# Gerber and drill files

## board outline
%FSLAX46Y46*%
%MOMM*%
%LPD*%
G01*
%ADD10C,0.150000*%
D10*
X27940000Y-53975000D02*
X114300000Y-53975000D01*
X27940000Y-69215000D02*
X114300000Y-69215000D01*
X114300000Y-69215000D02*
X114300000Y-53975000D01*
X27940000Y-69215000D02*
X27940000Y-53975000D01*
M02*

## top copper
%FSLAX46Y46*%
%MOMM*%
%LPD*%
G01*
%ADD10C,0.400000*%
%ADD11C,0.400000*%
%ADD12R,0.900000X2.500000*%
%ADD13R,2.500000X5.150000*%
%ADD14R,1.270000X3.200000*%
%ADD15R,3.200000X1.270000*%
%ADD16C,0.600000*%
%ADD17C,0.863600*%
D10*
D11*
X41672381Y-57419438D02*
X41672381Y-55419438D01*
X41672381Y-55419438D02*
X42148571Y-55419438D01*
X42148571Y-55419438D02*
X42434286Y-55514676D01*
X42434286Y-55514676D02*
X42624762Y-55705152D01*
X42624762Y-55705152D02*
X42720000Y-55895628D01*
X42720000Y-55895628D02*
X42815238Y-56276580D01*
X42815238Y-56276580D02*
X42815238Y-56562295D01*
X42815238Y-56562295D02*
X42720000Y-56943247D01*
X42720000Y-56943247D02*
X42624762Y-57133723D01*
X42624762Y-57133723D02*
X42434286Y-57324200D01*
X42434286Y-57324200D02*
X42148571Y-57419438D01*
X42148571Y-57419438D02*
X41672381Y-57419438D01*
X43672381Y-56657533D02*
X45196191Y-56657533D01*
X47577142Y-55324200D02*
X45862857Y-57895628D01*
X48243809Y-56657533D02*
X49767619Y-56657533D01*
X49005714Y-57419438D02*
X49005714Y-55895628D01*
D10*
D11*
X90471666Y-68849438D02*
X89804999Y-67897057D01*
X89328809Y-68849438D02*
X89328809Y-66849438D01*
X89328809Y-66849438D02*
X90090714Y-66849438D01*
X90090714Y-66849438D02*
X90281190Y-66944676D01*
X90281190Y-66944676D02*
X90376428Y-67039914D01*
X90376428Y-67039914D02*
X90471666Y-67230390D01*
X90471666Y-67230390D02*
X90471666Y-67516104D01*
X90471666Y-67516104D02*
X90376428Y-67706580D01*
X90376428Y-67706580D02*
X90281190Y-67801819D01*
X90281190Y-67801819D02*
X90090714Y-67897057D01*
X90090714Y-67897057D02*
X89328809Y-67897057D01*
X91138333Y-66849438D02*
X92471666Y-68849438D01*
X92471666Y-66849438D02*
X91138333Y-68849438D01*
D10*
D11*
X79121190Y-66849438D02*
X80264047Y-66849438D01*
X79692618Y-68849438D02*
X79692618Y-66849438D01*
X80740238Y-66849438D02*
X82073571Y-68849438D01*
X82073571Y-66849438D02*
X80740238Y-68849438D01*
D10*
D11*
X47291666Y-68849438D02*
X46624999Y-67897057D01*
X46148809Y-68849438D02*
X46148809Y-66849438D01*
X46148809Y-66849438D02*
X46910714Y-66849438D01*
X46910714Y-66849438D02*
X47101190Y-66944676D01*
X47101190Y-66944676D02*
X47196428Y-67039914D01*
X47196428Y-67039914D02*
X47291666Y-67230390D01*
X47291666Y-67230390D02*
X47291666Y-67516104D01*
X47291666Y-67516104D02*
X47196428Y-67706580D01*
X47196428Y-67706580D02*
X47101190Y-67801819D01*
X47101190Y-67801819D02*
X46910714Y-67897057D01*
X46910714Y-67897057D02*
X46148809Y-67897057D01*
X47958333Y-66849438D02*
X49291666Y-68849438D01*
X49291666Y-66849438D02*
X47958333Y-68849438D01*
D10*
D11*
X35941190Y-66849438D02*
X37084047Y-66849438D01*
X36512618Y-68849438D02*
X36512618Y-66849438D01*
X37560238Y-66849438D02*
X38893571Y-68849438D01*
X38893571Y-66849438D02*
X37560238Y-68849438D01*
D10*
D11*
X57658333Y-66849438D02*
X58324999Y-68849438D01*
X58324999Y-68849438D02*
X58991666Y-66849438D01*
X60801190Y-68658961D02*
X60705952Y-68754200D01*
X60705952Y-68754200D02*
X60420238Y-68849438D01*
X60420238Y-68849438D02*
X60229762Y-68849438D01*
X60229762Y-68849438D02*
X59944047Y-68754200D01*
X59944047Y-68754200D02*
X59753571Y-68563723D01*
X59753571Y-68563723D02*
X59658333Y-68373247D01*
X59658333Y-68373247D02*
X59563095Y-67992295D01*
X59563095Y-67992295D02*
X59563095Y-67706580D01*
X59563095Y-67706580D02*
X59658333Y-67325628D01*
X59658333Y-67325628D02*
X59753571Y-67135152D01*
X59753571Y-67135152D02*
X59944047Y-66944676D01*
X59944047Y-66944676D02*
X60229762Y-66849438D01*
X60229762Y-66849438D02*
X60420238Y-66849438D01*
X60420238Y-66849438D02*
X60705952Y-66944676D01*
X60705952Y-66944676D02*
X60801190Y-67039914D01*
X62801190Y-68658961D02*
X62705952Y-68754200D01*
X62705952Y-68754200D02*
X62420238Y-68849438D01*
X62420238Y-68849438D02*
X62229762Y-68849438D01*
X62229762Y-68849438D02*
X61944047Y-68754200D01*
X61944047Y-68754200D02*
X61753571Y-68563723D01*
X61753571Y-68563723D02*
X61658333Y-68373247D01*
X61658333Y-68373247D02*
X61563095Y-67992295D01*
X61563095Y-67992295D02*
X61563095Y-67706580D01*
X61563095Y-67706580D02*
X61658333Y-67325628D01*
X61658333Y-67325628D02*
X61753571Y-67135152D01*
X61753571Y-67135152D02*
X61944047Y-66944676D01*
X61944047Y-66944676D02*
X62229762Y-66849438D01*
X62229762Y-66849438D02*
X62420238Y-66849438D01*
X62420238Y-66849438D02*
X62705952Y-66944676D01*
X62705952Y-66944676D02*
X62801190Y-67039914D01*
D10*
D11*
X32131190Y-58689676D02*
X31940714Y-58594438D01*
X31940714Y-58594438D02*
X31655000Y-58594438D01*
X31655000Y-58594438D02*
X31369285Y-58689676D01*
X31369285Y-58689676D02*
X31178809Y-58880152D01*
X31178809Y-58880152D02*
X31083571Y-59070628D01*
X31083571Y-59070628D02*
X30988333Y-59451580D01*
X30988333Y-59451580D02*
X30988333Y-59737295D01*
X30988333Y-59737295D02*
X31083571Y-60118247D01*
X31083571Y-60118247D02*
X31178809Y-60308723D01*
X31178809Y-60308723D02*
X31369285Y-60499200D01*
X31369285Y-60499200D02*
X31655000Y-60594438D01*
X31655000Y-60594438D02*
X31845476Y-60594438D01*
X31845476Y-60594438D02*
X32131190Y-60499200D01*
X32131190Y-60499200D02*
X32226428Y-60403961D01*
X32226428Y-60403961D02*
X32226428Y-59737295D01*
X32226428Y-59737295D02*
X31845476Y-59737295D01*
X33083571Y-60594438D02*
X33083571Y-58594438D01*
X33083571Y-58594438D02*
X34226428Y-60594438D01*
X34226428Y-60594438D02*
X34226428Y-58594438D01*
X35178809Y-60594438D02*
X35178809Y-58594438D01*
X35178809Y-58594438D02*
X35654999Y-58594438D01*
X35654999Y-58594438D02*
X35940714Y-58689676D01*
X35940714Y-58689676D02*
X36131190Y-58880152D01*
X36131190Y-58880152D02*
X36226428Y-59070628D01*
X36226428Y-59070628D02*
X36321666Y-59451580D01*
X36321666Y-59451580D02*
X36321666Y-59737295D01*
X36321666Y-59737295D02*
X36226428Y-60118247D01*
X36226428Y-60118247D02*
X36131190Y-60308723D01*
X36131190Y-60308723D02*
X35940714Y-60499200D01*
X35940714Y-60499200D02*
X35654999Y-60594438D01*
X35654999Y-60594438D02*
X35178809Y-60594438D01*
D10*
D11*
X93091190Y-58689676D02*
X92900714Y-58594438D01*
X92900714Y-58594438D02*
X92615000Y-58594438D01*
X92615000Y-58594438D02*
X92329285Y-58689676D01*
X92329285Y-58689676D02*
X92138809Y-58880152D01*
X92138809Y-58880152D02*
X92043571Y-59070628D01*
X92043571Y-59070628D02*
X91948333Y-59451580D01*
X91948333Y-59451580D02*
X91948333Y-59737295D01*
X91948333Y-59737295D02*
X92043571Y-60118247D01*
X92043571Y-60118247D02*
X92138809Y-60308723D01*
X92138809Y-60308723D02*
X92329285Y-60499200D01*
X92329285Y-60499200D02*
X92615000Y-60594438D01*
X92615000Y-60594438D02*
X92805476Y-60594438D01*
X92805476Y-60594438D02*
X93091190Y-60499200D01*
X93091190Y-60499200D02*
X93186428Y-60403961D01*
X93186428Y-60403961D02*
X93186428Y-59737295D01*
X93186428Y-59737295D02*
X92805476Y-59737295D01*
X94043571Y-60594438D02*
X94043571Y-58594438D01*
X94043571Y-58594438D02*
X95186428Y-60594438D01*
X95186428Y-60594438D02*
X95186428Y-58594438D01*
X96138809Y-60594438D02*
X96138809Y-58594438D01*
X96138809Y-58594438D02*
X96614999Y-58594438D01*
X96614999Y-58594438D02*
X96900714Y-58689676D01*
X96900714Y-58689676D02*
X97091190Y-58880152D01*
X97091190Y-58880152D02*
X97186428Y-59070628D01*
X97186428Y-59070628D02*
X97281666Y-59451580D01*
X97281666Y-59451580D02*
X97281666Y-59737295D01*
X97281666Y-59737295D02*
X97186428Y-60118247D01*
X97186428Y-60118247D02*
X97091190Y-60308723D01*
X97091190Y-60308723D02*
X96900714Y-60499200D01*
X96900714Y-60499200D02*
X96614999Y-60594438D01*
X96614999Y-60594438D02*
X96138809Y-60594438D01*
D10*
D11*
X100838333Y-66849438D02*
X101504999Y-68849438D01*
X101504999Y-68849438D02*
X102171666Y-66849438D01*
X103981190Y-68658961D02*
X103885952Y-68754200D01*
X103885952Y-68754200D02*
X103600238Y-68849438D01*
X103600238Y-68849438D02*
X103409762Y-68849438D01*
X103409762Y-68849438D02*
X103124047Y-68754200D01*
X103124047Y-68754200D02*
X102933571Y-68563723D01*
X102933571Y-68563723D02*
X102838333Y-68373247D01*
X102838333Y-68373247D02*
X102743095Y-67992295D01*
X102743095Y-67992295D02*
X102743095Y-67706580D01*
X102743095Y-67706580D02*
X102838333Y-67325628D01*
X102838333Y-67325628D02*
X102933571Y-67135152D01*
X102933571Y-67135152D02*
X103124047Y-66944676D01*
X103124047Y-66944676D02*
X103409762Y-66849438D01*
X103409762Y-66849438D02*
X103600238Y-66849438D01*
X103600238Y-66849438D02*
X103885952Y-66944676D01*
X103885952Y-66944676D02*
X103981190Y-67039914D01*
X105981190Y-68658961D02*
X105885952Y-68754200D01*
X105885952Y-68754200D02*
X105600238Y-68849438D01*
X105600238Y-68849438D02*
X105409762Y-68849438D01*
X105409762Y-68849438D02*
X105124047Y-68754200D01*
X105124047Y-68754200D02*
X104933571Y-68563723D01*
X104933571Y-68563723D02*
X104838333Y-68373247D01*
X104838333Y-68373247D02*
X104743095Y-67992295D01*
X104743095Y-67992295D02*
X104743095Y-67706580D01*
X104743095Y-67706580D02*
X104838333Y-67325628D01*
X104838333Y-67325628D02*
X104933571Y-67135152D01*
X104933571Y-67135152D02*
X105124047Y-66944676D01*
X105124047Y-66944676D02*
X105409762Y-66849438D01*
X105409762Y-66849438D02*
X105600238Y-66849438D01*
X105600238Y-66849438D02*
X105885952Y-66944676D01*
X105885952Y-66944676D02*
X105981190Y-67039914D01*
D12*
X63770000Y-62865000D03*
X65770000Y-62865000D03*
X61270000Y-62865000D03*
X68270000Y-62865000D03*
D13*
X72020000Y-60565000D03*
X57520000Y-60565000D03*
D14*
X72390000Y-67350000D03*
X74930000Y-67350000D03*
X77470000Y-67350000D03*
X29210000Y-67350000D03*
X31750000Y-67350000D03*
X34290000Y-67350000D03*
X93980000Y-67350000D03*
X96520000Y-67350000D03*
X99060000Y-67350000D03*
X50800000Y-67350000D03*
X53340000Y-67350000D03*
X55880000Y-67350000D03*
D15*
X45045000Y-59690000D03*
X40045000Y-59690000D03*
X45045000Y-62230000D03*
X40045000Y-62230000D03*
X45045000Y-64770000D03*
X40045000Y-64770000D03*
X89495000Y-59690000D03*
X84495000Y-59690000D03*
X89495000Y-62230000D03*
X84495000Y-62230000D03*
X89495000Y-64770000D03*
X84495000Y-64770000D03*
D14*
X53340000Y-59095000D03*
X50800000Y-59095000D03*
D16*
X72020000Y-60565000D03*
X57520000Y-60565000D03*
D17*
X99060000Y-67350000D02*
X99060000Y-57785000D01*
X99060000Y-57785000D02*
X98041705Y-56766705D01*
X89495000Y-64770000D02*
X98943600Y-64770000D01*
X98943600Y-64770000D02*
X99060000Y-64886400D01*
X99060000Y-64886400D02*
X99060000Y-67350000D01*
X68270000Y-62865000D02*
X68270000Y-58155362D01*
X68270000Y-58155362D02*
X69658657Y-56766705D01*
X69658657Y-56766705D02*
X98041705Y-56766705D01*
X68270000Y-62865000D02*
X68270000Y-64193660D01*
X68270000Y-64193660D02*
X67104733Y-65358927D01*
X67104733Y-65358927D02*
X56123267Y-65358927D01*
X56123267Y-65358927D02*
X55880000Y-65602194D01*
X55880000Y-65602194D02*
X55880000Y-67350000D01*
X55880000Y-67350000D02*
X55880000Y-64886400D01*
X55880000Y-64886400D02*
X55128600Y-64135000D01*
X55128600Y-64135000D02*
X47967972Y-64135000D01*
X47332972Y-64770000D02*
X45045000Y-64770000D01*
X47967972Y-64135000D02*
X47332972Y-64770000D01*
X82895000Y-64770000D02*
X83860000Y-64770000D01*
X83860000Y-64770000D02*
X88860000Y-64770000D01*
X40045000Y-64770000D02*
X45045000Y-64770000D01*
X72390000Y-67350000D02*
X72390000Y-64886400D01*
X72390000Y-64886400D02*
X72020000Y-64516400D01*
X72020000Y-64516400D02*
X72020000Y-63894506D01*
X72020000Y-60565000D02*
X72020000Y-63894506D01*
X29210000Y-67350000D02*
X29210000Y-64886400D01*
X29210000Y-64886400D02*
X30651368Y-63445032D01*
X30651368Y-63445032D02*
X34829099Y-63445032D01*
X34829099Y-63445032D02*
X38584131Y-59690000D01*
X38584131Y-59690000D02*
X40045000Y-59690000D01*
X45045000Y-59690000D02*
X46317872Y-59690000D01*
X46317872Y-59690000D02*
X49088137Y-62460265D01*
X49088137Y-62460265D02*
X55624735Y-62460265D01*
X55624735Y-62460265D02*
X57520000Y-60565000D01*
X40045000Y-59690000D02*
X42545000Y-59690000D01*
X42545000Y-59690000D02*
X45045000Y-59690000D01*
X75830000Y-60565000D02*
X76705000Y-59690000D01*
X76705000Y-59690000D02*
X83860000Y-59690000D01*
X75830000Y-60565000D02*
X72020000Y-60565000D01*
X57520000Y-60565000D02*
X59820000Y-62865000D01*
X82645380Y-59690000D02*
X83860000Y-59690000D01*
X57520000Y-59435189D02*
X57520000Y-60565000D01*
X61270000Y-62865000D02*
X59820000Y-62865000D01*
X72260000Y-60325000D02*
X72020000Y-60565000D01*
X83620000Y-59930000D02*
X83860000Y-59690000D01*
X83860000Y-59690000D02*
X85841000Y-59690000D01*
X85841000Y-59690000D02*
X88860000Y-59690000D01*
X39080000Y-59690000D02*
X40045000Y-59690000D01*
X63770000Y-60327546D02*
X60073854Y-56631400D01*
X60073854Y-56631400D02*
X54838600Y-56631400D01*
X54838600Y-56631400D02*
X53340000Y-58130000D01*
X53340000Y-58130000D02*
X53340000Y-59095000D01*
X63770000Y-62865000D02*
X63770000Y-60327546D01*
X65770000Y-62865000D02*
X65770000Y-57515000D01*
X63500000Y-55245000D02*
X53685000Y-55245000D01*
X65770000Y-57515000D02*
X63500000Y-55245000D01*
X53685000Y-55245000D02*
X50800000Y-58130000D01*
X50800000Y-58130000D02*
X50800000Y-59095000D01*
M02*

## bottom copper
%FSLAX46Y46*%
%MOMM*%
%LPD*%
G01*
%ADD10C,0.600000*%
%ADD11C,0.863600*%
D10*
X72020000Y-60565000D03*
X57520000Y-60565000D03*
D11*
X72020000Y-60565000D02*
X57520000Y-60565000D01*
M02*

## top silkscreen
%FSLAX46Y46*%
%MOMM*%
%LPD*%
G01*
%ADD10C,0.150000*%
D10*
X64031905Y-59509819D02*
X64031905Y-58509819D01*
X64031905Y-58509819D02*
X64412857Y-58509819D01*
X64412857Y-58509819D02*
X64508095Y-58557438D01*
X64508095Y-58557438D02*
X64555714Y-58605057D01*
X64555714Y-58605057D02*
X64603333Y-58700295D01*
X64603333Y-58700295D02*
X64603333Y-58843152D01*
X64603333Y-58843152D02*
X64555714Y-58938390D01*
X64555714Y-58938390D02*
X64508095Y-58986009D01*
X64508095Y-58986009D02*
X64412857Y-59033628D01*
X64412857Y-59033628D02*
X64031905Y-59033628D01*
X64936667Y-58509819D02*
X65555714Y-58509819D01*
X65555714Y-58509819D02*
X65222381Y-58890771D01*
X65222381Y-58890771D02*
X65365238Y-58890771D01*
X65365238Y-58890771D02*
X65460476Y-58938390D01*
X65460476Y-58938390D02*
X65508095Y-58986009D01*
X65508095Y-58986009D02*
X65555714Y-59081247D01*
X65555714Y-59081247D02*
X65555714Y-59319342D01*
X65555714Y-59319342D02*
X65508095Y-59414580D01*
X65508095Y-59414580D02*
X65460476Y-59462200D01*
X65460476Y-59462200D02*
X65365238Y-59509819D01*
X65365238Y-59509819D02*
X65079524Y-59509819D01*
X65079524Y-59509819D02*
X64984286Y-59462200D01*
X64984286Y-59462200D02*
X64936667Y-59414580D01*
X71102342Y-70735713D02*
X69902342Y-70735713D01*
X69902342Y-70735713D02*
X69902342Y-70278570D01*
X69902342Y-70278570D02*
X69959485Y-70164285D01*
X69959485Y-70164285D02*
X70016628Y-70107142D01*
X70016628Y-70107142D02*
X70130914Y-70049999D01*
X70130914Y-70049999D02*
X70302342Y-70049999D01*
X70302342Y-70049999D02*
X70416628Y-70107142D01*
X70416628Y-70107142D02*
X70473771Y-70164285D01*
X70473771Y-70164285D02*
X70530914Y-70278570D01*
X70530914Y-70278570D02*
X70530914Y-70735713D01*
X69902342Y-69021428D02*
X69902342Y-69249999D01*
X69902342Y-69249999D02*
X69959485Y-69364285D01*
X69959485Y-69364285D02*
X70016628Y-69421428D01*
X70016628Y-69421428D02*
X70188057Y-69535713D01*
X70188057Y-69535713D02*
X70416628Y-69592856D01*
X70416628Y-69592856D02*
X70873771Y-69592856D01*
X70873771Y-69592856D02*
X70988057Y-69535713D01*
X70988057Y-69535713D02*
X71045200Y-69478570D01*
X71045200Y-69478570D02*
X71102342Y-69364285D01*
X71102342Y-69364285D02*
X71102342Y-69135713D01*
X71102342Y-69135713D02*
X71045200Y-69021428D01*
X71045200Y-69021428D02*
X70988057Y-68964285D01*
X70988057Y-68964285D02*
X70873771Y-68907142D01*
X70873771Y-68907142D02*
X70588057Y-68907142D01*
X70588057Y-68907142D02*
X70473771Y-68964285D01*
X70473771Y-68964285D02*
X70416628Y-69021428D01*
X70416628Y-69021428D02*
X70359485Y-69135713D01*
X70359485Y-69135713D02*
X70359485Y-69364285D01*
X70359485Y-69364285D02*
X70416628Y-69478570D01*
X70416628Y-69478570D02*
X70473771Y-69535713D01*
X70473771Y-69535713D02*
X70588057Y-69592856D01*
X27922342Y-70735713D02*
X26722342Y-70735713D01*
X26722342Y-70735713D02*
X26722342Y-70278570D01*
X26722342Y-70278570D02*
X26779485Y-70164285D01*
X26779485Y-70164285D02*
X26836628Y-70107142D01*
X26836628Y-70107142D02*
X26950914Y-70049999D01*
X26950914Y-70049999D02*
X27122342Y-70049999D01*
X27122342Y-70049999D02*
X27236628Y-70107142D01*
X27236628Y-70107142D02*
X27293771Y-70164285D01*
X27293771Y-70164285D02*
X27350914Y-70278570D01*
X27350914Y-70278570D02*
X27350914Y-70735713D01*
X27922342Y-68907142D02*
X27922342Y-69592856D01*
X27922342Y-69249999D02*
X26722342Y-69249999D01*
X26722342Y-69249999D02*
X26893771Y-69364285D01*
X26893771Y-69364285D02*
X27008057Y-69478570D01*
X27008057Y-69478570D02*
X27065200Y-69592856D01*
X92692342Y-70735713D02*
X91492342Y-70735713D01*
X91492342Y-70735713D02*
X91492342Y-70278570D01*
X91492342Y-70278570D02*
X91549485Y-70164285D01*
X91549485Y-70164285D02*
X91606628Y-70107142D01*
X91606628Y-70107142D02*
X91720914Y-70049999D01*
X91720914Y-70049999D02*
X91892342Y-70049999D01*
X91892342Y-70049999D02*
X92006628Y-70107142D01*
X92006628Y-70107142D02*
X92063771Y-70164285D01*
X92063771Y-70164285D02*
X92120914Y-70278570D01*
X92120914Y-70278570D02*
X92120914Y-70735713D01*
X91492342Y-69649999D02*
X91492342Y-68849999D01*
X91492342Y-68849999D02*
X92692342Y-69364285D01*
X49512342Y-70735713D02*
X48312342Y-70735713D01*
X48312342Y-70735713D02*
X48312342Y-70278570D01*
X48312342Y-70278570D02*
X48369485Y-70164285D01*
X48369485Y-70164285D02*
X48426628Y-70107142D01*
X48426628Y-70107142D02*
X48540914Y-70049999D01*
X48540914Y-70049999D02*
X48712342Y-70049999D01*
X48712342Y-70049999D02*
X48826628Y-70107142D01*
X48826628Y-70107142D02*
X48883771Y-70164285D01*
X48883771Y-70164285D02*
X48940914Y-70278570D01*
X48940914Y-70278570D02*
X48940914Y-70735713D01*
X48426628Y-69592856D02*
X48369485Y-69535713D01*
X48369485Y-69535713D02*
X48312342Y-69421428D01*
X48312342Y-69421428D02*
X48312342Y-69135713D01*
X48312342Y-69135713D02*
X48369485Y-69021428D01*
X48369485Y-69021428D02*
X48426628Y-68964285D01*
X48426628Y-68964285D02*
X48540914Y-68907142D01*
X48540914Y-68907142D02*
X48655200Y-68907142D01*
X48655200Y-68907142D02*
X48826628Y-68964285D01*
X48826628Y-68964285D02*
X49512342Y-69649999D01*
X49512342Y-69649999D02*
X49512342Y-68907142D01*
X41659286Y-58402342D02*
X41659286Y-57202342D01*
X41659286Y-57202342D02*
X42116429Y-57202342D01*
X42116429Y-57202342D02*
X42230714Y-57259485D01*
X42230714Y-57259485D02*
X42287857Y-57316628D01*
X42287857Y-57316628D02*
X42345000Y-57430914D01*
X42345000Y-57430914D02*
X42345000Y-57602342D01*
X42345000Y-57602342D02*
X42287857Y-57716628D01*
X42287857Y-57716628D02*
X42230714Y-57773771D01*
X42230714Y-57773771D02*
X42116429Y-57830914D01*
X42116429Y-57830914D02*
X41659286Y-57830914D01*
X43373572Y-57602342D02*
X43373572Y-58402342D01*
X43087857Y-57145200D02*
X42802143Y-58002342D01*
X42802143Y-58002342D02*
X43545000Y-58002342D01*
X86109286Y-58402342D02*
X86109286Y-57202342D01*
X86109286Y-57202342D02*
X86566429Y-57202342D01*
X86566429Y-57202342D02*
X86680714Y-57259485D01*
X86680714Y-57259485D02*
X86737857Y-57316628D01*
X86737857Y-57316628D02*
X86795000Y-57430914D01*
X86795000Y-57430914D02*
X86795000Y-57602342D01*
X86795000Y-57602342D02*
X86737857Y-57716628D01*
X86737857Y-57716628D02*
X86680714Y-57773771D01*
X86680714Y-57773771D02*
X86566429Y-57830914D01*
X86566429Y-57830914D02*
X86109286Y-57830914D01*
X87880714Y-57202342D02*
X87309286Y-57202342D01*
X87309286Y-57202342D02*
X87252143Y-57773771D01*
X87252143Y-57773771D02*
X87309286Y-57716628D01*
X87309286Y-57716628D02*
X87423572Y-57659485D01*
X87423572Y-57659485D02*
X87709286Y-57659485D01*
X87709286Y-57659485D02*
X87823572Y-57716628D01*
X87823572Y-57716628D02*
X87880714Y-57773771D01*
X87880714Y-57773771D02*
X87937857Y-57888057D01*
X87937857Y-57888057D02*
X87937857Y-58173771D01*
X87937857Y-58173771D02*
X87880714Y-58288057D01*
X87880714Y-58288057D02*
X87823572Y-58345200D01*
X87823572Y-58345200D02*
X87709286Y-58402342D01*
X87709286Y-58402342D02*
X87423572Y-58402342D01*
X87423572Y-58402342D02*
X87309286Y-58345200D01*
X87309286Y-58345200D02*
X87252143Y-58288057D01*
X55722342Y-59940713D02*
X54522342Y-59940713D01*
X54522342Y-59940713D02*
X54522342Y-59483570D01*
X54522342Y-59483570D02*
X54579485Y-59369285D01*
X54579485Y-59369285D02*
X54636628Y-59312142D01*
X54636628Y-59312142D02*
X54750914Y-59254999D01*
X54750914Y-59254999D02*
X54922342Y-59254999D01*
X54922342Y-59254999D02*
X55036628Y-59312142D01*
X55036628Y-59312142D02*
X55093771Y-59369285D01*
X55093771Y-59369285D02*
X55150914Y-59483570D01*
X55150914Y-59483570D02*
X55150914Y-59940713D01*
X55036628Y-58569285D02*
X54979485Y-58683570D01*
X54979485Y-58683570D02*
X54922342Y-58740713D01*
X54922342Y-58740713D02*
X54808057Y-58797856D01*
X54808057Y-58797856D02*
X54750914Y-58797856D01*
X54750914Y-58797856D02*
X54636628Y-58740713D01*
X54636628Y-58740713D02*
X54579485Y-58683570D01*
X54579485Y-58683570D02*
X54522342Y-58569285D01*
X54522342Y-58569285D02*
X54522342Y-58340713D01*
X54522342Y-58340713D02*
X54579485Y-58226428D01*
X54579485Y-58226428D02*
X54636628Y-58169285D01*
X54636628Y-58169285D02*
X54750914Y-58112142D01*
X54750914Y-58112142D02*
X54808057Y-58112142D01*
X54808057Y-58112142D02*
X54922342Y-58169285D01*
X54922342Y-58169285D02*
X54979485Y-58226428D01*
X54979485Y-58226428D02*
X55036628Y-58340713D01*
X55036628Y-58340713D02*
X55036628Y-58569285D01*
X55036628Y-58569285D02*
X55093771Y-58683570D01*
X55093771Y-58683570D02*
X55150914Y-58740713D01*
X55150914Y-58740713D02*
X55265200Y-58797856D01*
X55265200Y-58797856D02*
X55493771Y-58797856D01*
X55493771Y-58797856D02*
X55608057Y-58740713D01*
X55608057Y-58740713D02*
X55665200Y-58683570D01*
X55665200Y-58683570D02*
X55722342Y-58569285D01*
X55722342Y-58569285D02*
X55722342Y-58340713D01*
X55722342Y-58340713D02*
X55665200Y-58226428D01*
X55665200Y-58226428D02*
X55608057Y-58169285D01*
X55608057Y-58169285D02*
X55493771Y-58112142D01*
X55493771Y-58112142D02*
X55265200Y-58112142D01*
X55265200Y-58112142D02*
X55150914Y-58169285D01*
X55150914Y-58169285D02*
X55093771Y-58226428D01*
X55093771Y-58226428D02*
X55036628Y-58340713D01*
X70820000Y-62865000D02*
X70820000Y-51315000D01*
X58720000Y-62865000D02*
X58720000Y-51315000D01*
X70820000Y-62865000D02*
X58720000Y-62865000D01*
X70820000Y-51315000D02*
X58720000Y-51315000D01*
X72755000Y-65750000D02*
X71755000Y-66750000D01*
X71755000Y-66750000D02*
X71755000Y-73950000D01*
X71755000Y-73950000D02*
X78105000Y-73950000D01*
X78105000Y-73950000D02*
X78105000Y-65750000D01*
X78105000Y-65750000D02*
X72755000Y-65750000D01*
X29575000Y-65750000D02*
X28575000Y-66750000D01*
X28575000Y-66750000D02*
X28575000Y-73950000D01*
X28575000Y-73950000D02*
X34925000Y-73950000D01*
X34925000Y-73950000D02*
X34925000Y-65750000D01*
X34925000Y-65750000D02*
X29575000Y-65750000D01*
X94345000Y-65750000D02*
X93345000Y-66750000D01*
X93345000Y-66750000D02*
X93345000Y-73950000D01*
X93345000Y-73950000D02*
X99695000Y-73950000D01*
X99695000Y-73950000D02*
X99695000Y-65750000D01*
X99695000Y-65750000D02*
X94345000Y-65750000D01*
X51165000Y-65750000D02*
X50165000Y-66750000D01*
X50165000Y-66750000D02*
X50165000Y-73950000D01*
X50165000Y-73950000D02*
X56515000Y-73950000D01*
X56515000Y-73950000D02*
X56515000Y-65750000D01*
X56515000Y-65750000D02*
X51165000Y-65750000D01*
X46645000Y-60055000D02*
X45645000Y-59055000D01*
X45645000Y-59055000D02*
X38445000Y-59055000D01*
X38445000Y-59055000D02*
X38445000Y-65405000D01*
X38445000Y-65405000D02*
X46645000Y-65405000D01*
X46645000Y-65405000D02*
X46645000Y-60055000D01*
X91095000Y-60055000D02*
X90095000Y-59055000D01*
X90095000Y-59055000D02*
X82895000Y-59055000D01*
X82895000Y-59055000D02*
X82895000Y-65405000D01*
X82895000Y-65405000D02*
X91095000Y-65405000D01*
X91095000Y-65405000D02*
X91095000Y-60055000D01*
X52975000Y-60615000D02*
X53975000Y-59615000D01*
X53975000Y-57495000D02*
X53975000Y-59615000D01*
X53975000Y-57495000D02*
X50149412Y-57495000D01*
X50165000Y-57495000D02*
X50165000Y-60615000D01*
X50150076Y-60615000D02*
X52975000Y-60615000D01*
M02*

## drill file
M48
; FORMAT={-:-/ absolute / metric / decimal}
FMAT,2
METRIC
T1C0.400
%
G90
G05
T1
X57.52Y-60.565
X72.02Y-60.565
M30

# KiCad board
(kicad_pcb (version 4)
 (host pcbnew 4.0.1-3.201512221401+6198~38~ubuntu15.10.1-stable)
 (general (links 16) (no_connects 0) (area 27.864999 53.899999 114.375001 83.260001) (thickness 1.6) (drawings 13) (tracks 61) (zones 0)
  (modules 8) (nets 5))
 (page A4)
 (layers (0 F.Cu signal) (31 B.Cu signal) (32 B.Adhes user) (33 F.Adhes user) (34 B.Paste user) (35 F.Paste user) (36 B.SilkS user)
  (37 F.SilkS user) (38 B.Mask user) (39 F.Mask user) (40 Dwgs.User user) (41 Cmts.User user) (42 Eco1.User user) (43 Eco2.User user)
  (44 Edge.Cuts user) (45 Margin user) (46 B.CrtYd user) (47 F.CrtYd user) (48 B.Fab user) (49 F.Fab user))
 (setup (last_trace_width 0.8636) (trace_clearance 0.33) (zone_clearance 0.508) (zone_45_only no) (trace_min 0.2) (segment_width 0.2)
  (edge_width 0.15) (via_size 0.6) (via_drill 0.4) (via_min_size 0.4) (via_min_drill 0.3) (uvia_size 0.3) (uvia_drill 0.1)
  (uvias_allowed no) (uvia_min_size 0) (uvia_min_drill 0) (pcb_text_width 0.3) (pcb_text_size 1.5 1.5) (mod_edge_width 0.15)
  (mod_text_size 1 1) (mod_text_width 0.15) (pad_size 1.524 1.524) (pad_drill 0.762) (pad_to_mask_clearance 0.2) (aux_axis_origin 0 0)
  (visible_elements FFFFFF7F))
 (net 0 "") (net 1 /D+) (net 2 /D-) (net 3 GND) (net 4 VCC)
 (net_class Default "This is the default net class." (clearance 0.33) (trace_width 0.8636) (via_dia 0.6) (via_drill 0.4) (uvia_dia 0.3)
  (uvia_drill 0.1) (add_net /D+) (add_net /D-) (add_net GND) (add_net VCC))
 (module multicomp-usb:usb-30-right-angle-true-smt (layer F.Cu) (at 64.77 62.865 180)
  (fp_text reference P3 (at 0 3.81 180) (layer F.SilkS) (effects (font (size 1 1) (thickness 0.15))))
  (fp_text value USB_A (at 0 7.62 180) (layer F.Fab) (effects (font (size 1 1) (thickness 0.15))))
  (fp_line (start -6.05 0) (end -6.05 11.55) (layer F.SilkS) (width 0.15))
  (fp_line (start 6.05 0) (end 6.05 11.55) (layer F.SilkS) (width 0.15))
  (fp_line (start -6.05 0) (end 6.05 0) (layer F.SilkS) (width 0.15))
  (fp_line (start -6.05 11.55) (end 6.05 11.55) (layer F.SilkS) (width 0.15))
  (pad 3 smd rect (at 1 0 180) (size 0.9 2.5) (layers F.Cu F.Paste F.Mask) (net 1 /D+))
  (pad 2 smd rect (at -1 0 180) (size 0.9 2.5) (layers F.Cu F.Paste F.Mask) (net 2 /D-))
  (pad 4 smd rect (at 3.5 0 180) (size 0.9 2.5) (layers F.Cu F.Paste F.Mask) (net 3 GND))
  (pad 1 smd rect (at -3.5 0 180) (size 0.9 2.5) (layers F.Cu F.Paste F.Mask) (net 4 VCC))
  (pad 5 smd rect (at -7.25 2.3 180) (size 2.5 5.15) (layers F.Cu F.Paste F.Mask) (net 3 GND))
  (pad 5 smd rect (at 7.25 2.3 180) (size 2.5 5.15) (layers F.Cu F.Paste F.Mask) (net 3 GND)))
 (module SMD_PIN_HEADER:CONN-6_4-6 (layer F.Cu) (at 74.93 69.85)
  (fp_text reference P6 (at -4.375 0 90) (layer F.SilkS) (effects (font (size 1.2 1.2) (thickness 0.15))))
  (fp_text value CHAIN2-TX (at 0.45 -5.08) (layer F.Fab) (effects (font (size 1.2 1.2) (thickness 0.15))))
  (fp_line (start -2.175 -4.1) (end -3.175 -3.1) (layer F.SilkS) (width 0.15))
  (fp_line (start -3.175 -3.1) (end -3.175 4.1) (layer F.SilkS) (width 0.15))
  (fp_line (start -3.175 4.1) (end 3.175 4.1) (layer F.SilkS) (width 0.15))
  (fp_line (start 3.175 4.1) (end 3.175 -4.1) (layer F.SilkS) (width 0.15))
  (fp_line (start 3.175 -4.1) (end -2.175 -4.1) (layer F.SilkS) (width 0.15))
  (pad 6 smd rect (at -2.54 -2.5) (size 1.27 3.2) (layers F.Cu F.Paste F.Mask) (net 3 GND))
  (pad 5 smd rect (at 0 -2.5) (size 1.27 3.2) (layers F.Cu F.Paste F.Mask))
  (pad 4 smd rect (at 2.54 -2.5) (size 1.27 3.2) (layers F.Cu F.Paste F.Mask)))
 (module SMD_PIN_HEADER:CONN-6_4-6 (layer F.Cu) (at 31.75 69.85)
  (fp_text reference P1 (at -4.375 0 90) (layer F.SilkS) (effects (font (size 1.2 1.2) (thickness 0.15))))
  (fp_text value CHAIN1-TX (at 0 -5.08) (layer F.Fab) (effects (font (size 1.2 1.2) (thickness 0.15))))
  (fp_line (start -2.175 -4.1) (end -3.175 -3.1) (layer F.SilkS) (width 0.15))
  (fp_line (start -3.175 -3.1) (end -3.175 4.1) (layer F.SilkS) (width 0.15))
  (fp_line (start -3.175 4.1) (end 3.175 4.1) (layer F.SilkS) (width 0.15))
  (fp_line (start 3.175 4.1) (end 3.175 -4.1) (layer F.SilkS) (width 0.15))
  (fp_line (start 3.175 -4.1) (end -2.175 -4.1) (layer F.SilkS) (width 0.15))
  (pad 6 smd rect (at -2.54 -2.5) (size 1.27 3.2) (layers F.Cu F.Paste F.Mask) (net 3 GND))
  (pad 5 smd rect (at 0 -2.5) (size 1.27 3.2) (layers F.Cu F.Paste F.Mask))
  (pad 4 smd rect (at 2.54 -2.5) (size 1.27 3.2) (layers F.Cu F.Paste F.Mask)))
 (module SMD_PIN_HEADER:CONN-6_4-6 (layer F.Cu) (at 96.52 69.85)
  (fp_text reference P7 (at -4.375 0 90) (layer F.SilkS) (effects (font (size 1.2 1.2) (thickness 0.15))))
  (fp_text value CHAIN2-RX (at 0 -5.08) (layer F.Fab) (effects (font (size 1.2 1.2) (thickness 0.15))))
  (fp_line (start -2.175 -4.1) (end -3.175 -3.1) (layer F.SilkS) (width 0.15))
  (fp_line (start -3.175 -3.1) (end -3.175 4.1) (layer F.SilkS) (width 0.15))
  (fp_line (start -3.175 4.1) (end 3.175 4.1) (layer F.SilkS) (width 0.15))
  (fp_line (start 3.175 4.1) (end 3.175 -4.1) (layer F.SilkS) (width 0.15))
  (fp_line (start 3.175 -4.1) (end -2.175 -4.1) (layer F.SilkS) (width 0.15))
  (pad 6 smd rect (at -2.54 -2.5) (size 1.27 3.2) (layers F.Cu F.Paste F.Mask))
  (pad 5 smd rect (at 0 -2.5) (size 1.27 3.2) (layers F.Cu F.Paste F.Mask))
  (pad 4 smd rect (at 2.54 -2.5) (size 1.27 3.2) (layers F.Cu F.Paste F.Mask) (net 4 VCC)))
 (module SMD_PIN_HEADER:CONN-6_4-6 (layer F.Cu) (at 53.34 69.85)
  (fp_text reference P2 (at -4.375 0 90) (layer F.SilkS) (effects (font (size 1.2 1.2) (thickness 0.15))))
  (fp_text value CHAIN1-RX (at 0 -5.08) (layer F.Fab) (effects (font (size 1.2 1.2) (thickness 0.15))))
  (fp_line (start -2.175 -4.1) (end -3.175 -3.1) (layer F.SilkS) (width 0.15))
  (fp_line (start -3.175 -3.1) (end -3.175 4.1) (layer F.SilkS) (width 0.15))
  (fp_line (start -3.175 4.1) (end 3.175 4.1) (layer F.SilkS) (width 0.15))
  (fp_line (start 3.175 4.1) (end 3.175 -4.1) (layer F.SilkS) (width 0.15))
  (fp_line (start 3.175 -4.1) (end -2.175 -4.1) (layer F.SilkS) (width 0.15))
  (pad 6 smd rect (at -2.54 -2.5) (size 1.27 3.2) (layers F.Cu F.Paste F.Mask))
  (pad 5 smd rect (at 0 -2.5) (size 1.27 3.2) (layers F.Cu F.Paste F.Mask))
  (pad 4 smd rect (at 2.54 -2.5) (size 1.27 3.2) (layers F.Cu F.Paste F.Mask) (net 4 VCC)))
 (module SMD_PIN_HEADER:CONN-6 (layer F.Cu) (at 42.545 62.23 270)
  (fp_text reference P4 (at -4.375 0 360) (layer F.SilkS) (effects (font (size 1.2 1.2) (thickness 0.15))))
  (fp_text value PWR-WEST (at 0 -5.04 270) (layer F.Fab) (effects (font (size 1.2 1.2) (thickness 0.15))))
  (fp_line (start -2.175 -4.1) (end -3.175 -3.1) (layer F.SilkS) (width 0.15))
  (fp_line (start -3.175 -3.1) (end -3.175 4.1) (layer F.SilkS) (width 0.15))
  (fp_line (start -3.175 4.1) (end 3.175 4.1) (layer F.SilkS) (width 0.15))
  (fp_line (start 3.175 4.1) (end 3.175 -4.1) (layer F.SilkS) (width 0.15))
  (fp_line (start 3.175 -4.1) (end -2.175 -4.1) (layer F.SilkS) (width 0.15))
  (pad 6 smd rect (at -2.54 -2.5 270) (size 1.27 3.2) (layers F.Cu F.Paste F.Mask) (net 3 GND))
  (pad 1 smd rect (at -2.54 2.5 270) (size 1.27 3.2) (layers F.Cu F.Paste F.Mask) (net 3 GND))
  (pad 5 smd rect (at 0 -2.5 270) (size 1.27 3.2) (layers F.Cu F.Paste F.Mask))
  (pad 2 smd rect (at 0 2.5 270) (size 1.27 3.2) (layers F.Cu F.Paste F.Mask))
  (pad 4 smd rect (at 2.54 -2.5 270) (size 1.27 3.2) (layers F.Cu F.Paste F.Mask) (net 4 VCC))
  (pad 3 smd rect (at 2.54 2.5 270) (size 1.27 3.2) (layers F.Cu F.Paste F.Mask) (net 4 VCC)))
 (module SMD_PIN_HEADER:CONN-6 (layer F.Cu) (at 86.995 62.23 270)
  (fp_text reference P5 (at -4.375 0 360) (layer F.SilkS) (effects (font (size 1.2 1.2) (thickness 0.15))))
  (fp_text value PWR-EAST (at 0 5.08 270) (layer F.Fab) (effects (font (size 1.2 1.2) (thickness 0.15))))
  (fp_line (start -2.175 -4.1) (end -3.175 -3.1) (layer F.SilkS) (width 0.15))
  (fp_line (start -3.175 -3.1) (end -3.175 4.1) (layer F.SilkS) (width 0.15))
  (fp_line (start -3.175 4.1) (end 3.175 4.1) (layer F.SilkS) (width 0.15))
  (fp_line (start 3.175 4.1) (end 3.175 -4.1) (layer F.SilkS) (width 0.15))
  (fp_line (start 3.175 -4.1) (end -2.175 -4.1) (layer F.SilkS) (width 0.15))
  (pad 6 smd rect (at -2.54 -2.5 270) (size 1.27 3.2) (layers F.Cu F.Paste F.Mask) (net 3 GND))
  (pad 1 smd rect (at -2.54 2.5 270) (size 1.27 3.2) (layers F.Cu F.Paste F.Mask) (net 3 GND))
  (pad 5 smd rect (at 0 -2.5 270) (size 1.27 3.2) (layers F.Cu F.Paste F.Mask))
  (pad 2 smd rect (at 0 2.5 270) (size 1.27 3.2) (layers F.Cu F.Paste F.Mask))
  (pad 4 smd rect (at 2.54 -2.5 270) (size 1.27 3.2) (layers F.Cu F.Paste F.Mask) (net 4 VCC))
  (pad 3 smd rect (at 2.54 2.5 270) (size 1.27 3.2) (layers F.Cu F.Paste F.Mask) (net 4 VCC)))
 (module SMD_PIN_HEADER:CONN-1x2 (layer F.Cu) (at 52.07 59.055 180)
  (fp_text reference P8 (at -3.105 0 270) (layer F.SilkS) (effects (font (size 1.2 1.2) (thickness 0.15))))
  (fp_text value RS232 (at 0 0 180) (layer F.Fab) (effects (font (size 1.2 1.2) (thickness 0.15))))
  (fp_line (start -0.905 -1.56) (end -1.905 -0.56) (layer F.SilkS) (width 0.15))
  (fp_line (start -1.905 1.56) (end -1.905 -0.56) (layer F.SilkS) (width 0.15))
  (fp_line (start -1.905 1.56) (end 1.920588 1.56) (layer F.SilkS) (width 0.15))
  (fp_line (start 1.905 1.56) (end 1.905 -1.56) (layer F.SilkS) (width 0.15))
  (fp_line (start 1.919924 -1.56) (end -0.905 -1.56) (layer F.SilkS) (width 0.15))
  (pad 1 smd rect (at -1.27 -0.04 180) (size 1.27 3.2) (layers F.Cu F.Paste F.Mask) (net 1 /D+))
  (pad 2 smd rect (at 1.27 -0.04 180) (size 1.27 3.2) (layers F.Cu F.Paste F.Mask) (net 2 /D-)))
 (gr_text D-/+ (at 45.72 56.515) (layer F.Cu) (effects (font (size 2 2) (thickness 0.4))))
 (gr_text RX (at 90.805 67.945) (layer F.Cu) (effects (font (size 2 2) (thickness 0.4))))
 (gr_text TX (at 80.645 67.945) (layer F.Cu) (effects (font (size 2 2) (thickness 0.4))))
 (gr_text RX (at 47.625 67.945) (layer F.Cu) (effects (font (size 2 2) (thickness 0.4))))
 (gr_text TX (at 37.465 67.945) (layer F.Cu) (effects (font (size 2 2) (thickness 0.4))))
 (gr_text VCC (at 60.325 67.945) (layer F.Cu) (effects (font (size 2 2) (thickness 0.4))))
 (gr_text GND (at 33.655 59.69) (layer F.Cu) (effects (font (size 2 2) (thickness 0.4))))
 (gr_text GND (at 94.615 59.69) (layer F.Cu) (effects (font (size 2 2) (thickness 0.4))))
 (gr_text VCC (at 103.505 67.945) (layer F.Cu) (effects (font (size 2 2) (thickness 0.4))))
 (gr_line (start 27.94 53.975) (end 114.3 53.975) (layer Edge.Cuts) (width 0.15))
 (gr_line (start 27.94 69.215) (end 114.3 69.215) (layer Edge.Cuts) (width 0.15))
 (gr_line (start 114.3 69.215) (end 114.3 53.975) (layer Edge.Cuts) (width 0.15))
 (gr_line (start 27.94 69.215) (end 27.94 53.975) (layer Edge.Cuts) (width 0.15))
 (segment (start 99.06 67.35) (end 99.06 57.785) (width 0.8636) (layer F.Cu) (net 4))
 (segment (start 99.06 57.785) (end 98.041705 56.766705) (width 0.8636) (layer F.Cu) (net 4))
 (segment (start 89.495 64.77) (end 98.9436 64.77) (width 0.8636) (layer F.Cu) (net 4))
 (segment (start 98.9436 64.77) (end 99.06 64.8864) (width 0.8636) (layer F.Cu) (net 4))
 (segment (start 99.06 64.8864) (end 99.06 67.35) (width 0.8636) (layer F.Cu) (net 4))
 (segment (start 68.27 62.865) (end 68.27 58.155362) (width 0.8636) (layer F.Cu) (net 4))
 (segment (start 68.27 58.155362) (end 69.658657 56.766705) (width 0.8636) (layer F.Cu) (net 4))
 (segment (start 69.658657 56.766705) (end 98.041705 56.766705) (width 0.8636) (layer F.Cu) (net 4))
 (segment (start 68.27 62.865) (end 68.27 64.19366) (width 0.8636) (layer F.Cu) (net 4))
 (segment (start 68.27 64.19366) (end 67.104733 65.358927) (width 0.8636) (layer F.Cu) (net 4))
 (segment (start 67.104733 65.358927) (end 56.123267 65.358927) (width 0.8636) (layer F.Cu) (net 4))
 (segment (start 56.123267 65.358927) (end 55.88 65.602194) (width 0.8636) (layer F.Cu) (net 4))
 (segment (start 55.88 65.602194) (end 55.88 67.35) (width 0.8636) (layer F.Cu) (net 4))
 (segment (start 55.88 67.35) (end 55.88 64.8864) (width 0.8636) (layer F.Cu) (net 4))
 (segment (start 55.88 64.8864) (end 55.1286 64.135) (width 0.8636) (layer F.Cu) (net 4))
 (segment (start 55.1286 64.135) (end 47.967972 64.135) (width 0.8636) (layer F.Cu) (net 4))
 (segment (start 47.332972 64.77) (end 45.045 64.77) (width 0.8636) (layer F.Cu) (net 4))
 (segment (start 47.967972 64.135) (end 47.332972 64.77) (width 0.8636) (layer F.Cu) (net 4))
 (segment (start 82.895 64.77) (end 83.86 64.77) (width 0.8636) (layer F.Cu) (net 4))
 (segment (start 83.86 64.77) (end 88.86 64.77) (width 0.8636) (layer F.Cu) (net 4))
 (segment (start 40.045 64.77) (end 45.045 64.77) (width 0.8636) (layer F.Cu) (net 4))
 (segment (start 72.39 67.35) (end 72.39 64.8864) (width 0.8636) (layer F.Cu) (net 3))
 (segment (start 72.39 64.8864) (end 72.02 64.5164) (width 0.8636) (layer F.Cu) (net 3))
 (segment (start 72.02 64.5164) (end 72.02 63.894506) (width 0.8636) (layer F.Cu) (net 3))
 (segment (start 72.02 60.565) (end 72.02 63.894506) (width 0.8636) (layer F.Cu) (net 3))
 (segment (start 29.21 67.35) (end 29.21 64.8864) (width 0.8636) (layer F.Cu) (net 3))
 (segment (start 29.21 64.8864) (end 30.651368 63.445032) (width 0.8636) (layer F.Cu) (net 3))
 (segment (start 30.651368 63.445032) (end 34.829099 63.445032) (width 0.8636) (layer F.Cu) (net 3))
 (segment (start 34.829099 63.445032) (end 38.584131 59.69) (width 0.8636) (layer F.Cu) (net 3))
 (segment (start 38.584131 59.69) (end 40.045 59.69) (width 0.8636) (layer F.Cu) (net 3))
 (segment (start 45.045 59.69) (end 46.317872 59.69) (width 0.8636) (layer F.Cu) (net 3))
 (segment (start 46.317872 59.69) (end 49.088137 62.460265) (width 0.8636) (layer F.Cu) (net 3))
 (segment (start 49.088137 62.460265) (end 55.624735 62.460265) (width 0.8636) (layer F.Cu) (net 3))
 (segment (start 55.624735 62.460265) (end 57.52 60.565) (width 0.8636) (layer F.Cu) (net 3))
 (segment (start 40.045 59.69) (end 42.545 59.69) (width 0.8636) (layer F.Cu) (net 3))
 (segment (start 42.545 59.69) (end 45.045 59.69) (width 0.8636) (layer F.Cu) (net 3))
 (segment (start 75.83 60.565) (end 76.705 59.69) (width 0.8636) (layer F.Cu) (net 3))
 (segment (start 76.705 59.69) (end 83.86 59.69) (width 0.8636) (layer F.Cu) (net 3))
 (segment (start 75.83 60.565) (end 72.02 60.565) (width 0.8636) (layer F.Cu) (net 3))
 (segment (start 57.52 60.565) (end 59.82 62.865) (width 0.8636) (layer F.Cu) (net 3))
 (segment (start 82.64538 59.69) (end 83.86 59.69) (width 0.8636) (layer F.Cu) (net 3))
 (segment (start 57.52 59.435189) (end 57.52 60.565) (width 0.8636) (layer F.Cu) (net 3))
 (segment (start 72.02 60.565) (end 57.52 60.565) (width 0.8636) (layer B.Cu) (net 3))
 (via (at 72.02 60.565) (size 0.6) (drill 0.4) (layers F.Cu B.Cu) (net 3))
 (via (at 57.52 60.565) (size 0.6) (drill 0.4) (layers F.Cu B.Cu) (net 3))
 (segment (start 61.27 62.865) (end 59.82 62.865) (width 0.8636) (layer F.Cu) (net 3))
 (segment (start 72.26 60.325) (end 72.02 60.565) (width 0.8636) (layer F.Cu) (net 3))
 (segment (start 83.62 59.93) (end 83.86 59.69) (width 0.8636) (layer F.Cu) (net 3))
 (segment (start 83.86 59.69) (end 85.841 59.69) (width 0.8636) (layer F.Cu) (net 3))
 (segment (start 85.841 59.69) (end 88.86 59.69) (width 0.8636) (layer F.Cu) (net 3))
 (segment (start 39.08 59.69) (end 40.045 59.69) (width 0.8636) (layer F.Cu) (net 3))
 (segment (start 63.77 60.327546) (end 60.073854 56.6314) (width 0.8636) (layer F.Cu) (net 1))
 (segment (start 60.073854 56.6314) (end 54.8386 56.6314) (width 0.8636) (layer F.Cu) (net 1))
 (segment (start 54.8386 56.6314) (end 53.34 58.13) (width 0.8636) (layer F.Cu) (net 1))
 (segment (start 53.34 58.13) (end 53.34 59.095) (width 0.8636) (layer F.Cu) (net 1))
 (segment (start 63.77 62.865) (end 63.77 60.327546) (width 0.8636) (layer F.Cu) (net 1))
 (segment (start 65.77 62.865) (end 65.77 57.515) (width 0.8636) (layer F.Cu) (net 2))
 (segment (start 63.5 55.245) (end 53.685 55.245) (width 0.8636) (layer F.Cu) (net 2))
 (segment (start 65.77 57.515) (end 63.5 55.245) (width 0.8636) (layer F.Cu) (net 2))
 (segment (start 53.685 55.245) (end 50.8 58.13) (width 0.8636) (layer F.Cu) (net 2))
 (segment (start 50.8 58.13) (end 50.8 59.095) (width 0.8636) (layer F.Cu) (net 2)))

